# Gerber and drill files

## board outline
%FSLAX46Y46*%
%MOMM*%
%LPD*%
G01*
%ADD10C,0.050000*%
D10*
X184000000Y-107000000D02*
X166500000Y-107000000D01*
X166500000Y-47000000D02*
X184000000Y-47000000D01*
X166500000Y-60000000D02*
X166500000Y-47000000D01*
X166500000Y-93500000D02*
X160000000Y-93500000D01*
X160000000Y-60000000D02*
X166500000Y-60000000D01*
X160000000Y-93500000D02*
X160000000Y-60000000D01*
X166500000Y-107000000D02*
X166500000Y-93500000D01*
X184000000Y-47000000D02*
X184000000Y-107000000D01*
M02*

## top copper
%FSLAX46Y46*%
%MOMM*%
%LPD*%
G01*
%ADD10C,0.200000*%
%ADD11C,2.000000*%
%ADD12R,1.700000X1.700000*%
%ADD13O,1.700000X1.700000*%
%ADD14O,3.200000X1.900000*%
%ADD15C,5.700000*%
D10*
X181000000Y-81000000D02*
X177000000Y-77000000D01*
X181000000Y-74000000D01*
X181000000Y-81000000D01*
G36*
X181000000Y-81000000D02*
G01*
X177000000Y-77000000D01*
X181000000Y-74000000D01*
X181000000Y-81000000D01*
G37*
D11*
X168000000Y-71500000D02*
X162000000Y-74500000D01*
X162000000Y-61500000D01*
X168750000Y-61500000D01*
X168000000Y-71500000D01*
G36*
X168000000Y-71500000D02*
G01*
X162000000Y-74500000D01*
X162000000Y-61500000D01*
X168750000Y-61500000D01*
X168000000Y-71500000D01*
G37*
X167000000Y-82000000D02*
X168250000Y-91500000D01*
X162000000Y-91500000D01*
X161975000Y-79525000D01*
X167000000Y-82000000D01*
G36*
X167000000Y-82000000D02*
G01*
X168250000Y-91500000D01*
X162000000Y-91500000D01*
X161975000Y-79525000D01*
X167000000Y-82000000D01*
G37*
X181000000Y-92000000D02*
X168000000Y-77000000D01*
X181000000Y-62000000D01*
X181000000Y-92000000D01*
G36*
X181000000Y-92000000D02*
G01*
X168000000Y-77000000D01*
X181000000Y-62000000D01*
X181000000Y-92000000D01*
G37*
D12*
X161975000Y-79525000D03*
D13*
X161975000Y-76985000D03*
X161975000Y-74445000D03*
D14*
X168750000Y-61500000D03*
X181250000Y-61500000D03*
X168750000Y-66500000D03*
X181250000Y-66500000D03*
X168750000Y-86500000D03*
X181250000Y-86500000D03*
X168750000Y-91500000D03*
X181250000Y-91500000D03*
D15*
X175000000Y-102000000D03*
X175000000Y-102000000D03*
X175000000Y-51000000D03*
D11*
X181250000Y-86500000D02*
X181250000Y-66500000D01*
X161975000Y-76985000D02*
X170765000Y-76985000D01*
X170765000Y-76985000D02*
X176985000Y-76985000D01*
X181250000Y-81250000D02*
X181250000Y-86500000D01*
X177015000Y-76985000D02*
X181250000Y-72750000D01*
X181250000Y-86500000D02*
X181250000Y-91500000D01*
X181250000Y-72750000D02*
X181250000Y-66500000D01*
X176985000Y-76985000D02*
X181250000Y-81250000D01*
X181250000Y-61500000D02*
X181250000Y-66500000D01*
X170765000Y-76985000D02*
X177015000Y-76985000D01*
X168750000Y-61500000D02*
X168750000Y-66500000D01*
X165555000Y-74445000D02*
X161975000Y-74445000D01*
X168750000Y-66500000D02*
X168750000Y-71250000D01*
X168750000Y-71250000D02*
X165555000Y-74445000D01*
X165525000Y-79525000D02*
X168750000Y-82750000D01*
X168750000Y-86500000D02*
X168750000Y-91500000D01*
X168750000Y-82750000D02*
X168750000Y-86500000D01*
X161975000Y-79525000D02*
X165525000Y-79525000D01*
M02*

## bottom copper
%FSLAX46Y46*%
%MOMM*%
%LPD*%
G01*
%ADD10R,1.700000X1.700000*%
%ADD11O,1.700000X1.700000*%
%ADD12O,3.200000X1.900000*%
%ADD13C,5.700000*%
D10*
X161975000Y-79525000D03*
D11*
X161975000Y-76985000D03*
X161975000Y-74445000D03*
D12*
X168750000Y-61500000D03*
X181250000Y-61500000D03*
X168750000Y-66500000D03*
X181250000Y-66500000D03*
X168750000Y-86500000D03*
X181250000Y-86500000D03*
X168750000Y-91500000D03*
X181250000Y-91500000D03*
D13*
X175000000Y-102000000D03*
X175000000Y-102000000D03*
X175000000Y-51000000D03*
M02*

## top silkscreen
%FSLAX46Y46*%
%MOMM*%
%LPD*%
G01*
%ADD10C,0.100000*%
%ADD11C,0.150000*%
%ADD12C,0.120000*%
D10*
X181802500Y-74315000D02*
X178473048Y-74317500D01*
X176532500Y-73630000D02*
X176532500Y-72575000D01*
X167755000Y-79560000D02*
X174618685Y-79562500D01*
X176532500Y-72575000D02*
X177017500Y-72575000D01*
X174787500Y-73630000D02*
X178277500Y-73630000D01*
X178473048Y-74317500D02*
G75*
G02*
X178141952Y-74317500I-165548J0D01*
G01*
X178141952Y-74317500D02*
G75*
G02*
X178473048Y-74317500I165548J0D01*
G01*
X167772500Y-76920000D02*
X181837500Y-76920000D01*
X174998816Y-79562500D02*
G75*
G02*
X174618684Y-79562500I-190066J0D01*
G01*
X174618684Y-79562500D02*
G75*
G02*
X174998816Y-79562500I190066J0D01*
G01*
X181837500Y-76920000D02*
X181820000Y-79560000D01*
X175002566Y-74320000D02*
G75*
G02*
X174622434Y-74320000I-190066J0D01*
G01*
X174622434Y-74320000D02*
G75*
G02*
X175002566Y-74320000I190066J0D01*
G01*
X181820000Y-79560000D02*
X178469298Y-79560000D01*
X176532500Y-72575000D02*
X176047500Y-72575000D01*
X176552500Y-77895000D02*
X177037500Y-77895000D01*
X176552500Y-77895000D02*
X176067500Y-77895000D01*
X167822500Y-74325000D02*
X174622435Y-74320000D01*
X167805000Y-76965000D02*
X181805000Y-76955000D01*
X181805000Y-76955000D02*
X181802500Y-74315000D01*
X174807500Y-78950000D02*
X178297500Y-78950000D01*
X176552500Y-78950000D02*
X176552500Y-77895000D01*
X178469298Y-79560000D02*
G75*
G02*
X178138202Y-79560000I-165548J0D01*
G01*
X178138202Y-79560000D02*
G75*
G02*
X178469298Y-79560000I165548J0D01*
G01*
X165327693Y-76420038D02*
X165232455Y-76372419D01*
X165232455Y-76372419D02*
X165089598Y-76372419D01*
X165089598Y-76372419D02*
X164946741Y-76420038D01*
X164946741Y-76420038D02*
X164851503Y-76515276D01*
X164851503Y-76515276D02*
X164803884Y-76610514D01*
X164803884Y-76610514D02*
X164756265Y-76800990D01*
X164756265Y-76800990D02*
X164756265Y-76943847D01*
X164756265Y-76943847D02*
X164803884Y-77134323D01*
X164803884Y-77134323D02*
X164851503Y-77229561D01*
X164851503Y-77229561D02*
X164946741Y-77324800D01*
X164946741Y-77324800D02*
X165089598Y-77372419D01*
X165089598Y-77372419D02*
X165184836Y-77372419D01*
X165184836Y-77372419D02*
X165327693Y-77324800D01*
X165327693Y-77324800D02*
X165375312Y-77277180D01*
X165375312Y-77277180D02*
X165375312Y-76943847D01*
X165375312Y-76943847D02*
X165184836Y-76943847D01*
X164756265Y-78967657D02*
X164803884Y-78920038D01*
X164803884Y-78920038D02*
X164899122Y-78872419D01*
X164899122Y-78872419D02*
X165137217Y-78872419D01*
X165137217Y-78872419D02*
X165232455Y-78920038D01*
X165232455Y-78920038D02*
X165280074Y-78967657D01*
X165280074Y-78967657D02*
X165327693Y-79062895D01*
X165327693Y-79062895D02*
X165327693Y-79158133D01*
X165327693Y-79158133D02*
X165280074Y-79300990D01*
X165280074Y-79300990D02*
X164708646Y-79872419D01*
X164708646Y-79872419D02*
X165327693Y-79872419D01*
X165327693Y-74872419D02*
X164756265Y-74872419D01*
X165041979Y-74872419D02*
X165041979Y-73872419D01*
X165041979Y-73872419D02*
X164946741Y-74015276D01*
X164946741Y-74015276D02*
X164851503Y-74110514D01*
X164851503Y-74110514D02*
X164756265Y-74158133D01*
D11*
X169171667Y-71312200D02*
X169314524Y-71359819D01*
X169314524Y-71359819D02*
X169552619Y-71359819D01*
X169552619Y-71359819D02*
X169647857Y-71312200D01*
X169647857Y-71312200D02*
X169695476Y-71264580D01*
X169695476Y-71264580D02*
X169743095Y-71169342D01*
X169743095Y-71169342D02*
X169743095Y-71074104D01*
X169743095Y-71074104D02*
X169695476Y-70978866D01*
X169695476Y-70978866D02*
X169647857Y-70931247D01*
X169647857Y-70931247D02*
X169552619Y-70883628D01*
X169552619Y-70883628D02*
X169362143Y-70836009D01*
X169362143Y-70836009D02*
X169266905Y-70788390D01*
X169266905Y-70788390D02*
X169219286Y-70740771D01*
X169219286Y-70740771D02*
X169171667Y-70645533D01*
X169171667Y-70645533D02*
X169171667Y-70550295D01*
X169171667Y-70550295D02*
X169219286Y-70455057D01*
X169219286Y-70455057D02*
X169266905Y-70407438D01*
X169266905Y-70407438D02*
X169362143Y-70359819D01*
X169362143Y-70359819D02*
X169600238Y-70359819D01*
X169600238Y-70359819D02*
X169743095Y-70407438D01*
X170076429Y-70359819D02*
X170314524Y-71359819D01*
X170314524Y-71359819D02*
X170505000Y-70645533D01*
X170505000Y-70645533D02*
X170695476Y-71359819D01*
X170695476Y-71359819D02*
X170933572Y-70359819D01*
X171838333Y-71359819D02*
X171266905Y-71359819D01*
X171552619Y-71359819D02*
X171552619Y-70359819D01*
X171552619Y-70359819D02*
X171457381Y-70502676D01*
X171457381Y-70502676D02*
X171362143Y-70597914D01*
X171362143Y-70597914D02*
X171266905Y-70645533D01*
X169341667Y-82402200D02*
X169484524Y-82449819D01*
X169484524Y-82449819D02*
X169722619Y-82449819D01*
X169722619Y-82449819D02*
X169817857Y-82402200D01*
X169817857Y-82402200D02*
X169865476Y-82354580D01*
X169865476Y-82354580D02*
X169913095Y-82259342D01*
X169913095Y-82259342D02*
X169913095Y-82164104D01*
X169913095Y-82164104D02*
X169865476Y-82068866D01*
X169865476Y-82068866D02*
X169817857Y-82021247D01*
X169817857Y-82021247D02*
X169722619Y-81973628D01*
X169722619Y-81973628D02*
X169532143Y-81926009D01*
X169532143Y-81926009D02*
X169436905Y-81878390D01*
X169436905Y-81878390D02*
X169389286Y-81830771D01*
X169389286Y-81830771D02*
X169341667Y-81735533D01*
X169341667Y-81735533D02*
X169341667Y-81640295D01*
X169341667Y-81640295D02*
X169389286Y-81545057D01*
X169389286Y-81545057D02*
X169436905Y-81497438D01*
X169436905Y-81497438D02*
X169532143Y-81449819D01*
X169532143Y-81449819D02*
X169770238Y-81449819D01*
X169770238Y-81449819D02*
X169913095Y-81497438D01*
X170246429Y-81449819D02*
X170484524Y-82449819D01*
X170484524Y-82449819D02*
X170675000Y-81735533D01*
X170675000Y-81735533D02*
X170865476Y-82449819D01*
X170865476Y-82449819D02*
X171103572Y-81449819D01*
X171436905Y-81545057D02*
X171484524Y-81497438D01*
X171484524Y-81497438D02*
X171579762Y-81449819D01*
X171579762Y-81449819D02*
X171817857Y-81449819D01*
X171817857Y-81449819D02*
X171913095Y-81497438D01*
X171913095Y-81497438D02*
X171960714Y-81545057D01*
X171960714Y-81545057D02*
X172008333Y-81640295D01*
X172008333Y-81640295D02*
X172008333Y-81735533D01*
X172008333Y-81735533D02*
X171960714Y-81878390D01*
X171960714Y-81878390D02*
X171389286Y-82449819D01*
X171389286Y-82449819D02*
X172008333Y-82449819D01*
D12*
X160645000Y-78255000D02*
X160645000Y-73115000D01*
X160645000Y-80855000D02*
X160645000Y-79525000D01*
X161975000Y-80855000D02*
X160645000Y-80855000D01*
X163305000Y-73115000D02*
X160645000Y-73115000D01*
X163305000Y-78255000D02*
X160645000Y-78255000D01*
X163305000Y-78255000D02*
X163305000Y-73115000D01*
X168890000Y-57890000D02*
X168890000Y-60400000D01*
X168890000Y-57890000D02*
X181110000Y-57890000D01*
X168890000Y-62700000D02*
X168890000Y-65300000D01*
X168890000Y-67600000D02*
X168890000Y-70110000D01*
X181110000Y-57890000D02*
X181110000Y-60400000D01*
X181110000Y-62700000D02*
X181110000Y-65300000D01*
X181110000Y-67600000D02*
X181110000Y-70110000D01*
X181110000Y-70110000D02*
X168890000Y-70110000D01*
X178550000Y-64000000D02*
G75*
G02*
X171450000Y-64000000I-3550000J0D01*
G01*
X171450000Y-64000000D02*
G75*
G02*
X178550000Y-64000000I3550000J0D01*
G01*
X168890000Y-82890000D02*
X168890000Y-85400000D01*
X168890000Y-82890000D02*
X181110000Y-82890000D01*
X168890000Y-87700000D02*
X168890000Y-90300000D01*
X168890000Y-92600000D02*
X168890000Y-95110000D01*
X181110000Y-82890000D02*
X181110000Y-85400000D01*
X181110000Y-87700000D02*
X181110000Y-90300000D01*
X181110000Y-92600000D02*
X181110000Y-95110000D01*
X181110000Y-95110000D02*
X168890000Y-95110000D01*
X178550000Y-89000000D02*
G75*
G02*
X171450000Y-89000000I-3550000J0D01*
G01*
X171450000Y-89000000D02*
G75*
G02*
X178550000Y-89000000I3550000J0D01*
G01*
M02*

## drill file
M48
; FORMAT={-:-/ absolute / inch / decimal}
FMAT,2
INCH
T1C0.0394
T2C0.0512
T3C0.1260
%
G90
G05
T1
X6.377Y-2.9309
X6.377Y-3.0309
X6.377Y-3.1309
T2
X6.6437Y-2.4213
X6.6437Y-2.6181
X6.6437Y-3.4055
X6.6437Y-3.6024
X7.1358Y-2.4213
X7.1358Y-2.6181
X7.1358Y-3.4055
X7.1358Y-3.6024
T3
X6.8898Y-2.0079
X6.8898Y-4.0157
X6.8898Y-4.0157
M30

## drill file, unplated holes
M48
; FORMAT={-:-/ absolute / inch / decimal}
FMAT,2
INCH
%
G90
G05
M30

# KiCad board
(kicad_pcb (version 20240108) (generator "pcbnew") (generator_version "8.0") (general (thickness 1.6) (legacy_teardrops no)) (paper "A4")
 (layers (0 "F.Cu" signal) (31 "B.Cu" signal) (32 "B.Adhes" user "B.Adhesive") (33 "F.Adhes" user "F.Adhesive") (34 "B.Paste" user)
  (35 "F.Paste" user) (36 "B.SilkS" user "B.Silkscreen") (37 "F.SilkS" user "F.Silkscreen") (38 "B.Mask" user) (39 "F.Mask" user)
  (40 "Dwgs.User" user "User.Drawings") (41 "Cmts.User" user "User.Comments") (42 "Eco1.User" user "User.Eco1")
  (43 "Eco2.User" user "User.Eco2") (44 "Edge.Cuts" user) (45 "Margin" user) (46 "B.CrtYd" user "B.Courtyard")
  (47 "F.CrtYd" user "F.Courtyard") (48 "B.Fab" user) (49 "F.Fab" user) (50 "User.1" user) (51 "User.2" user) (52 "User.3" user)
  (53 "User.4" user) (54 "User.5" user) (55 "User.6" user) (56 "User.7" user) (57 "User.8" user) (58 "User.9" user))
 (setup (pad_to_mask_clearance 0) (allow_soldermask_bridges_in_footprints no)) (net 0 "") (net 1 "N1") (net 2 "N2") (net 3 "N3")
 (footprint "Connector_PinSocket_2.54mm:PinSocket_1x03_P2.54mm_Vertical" (layer "F.Cu") (at 161.975 79.525 180)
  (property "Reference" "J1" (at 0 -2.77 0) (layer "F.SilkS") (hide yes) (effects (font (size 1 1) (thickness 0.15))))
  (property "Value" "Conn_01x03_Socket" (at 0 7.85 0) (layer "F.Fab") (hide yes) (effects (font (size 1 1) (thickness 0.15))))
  (fp_line (start 1.33 1.27) (end 1.33 6.41) (stroke (width 0.12) (type solid)) (layer "F.SilkS"))
  (fp_line (start 1.33 -1.33) (end 1.33 0) (stroke (width 0.12) (type solid)) (layer "F.SilkS"))
  (fp_line (start 0 -1.33) (end 1.33 -1.33) (stroke (width 0.12) (type solid)) (layer "F.SilkS"))
  (fp_line (start -1.33 6.41) (end 1.33 6.41) (stroke (width 0.12) (type solid)) (layer "F.SilkS"))
  (fp_line (start -1.33 1.27) (end 1.33 1.27) (stroke (width 0.12) (type solid)) (layer "F.SilkS"))
  (fp_line (start -1.33 1.27) (end -1.33 6.41) (stroke (width 0.12) (type solid)) (layer "F.SilkS"))
  (pad "1" thru_hole rect (at 0 0 180) (size 1.7 1.7) (drill 1) (layers "*.Cu" "*.Mask") (remove_unused_layers no) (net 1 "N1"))
  (pad "2" thru_hole oval (at 0 2.54 180) (size 1.7 1.7) (drill 1) (layers "*.Cu" "*.Mask") (remove_unused_layers no) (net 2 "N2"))
  (pad "3" thru_hole oval (at 0 5.08 180) (size 1.7 1.7) (drill 1) (layers "*.Cu" "*.Mask") (remove_unused_layers no) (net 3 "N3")))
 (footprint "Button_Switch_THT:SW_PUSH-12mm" (layer "F.Cu") (at 168.75 61.5)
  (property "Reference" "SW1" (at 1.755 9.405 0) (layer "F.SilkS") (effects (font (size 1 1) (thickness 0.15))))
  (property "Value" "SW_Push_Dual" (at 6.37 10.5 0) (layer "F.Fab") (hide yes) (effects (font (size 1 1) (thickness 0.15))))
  (fp_line (start 0.14 -3.61) (end 0.14 -1.1) (stroke (width 0.12) (type default)) (layer "F.SilkS"))
  (fp_line (start 0.14 -3.61) (end 12.36 -3.61) (stroke (width 0.12) (type default)) (layer "F.SilkS"))
  (fp_line (start 0.14 1.2) (end 0.14 3.8) (stroke (width 0.12) (type default)) (layer "F.SilkS"))
  (fp_line (start 0.14 6.1) (end 0.14 8.61) (stroke (width 0.12) (type default)) (layer "F.SilkS"))
  (fp_line (start 12.36 -3.61) (end 12.36 -1.1) (stroke (width 0.12) (type default)) (layer "F.SilkS"))
  (fp_line (start 12.36 1.2) (end 12.36 3.8) (stroke (width 0.12) (type default)) (layer "F.SilkS"))
  (fp_line (start 12.36 6.1) (end 12.36 8.61) (stroke (width 0.12) (type default)) (layer "F.SilkS"))
  (fp_line (start 12.36 8.61) (end 0.14 8.61) (stroke (width 0.12) (type default)) (layer "F.SilkS"))
  (fp_circle (center 6.25 2.5) (end 9.8 2.5) (stroke (width 0.12) (type default)) (fill none) (layer "F.SilkS"))
  (pad "1" thru_hole oval (at 0 0) (size 3.2 1.9) (drill 1.3) (layers "*.Cu" "*.Mask") (remove_unused_layers no) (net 3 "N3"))
  (pad "2" thru_hole oval (at 12.5 0) (size 3.2 1.9) (drill 1.3) (layers "*.Cu" "*.Mask") (remove_unused_layers no) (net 2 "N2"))
  (pad "3" thru_hole oval (at 0 5) (size 3.2 1.9) (drill 1.3) (layers "*.Cu" "*.Mask") (remove_unused_layers no) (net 3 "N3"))
  (pad "4" thru_hole oval (at 12.5 5) (size 3.2 1.9) (drill 1.3) (layers "*.Cu" "*.Mask") (remove_unused_layers no) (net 2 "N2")))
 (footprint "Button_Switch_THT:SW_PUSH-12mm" (layer "F.Cu") (at 168.75 86.5)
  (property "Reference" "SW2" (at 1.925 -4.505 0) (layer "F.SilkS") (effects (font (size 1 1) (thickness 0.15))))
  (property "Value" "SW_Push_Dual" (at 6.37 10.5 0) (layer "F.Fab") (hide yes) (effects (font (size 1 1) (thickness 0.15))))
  (fp_line (start 0.14 -3.61) (end 0.14 -1.1) (stroke (width 0.12) (type default)) (layer "F.SilkS"))
  (fp_line (start 0.14 -3.61) (end 12.36 -3.61) (stroke (width 0.12) (type default)) (layer "F.SilkS"))
  (fp_line (start 0.14 1.2) (end 0.14 3.8) (stroke (width 0.12) (type default)) (layer "F.SilkS"))
  (fp_line (start 0.14 6.1) (end 0.14 8.61) (stroke (width 0.12) (type default)) (layer "F.SilkS"))
  (fp_line (start 12.36 -3.61) (end 12.36 -1.1) (stroke (width 0.12) (type default)) (layer "F.SilkS"))
  (fp_line (start 12.36 1.2) (end 12.36 3.8) (stroke (width 0.12) (type default)) (layer "F.SilkS"))
  (fp_line (start 12.36 6.1) (end 12.36 8.61) (stroke (width 0.12) (type default)) (layer "F.SilkS"))
  (fp_line (start 12.36 8.61) (end 0.14 8.61) (stroke (width 0.12) (type default)) (layer "F.SilkS"))
  (fp_circle (center 6.25 2.5) (end 9.8 2.5) (stroke (width 0.12) (type default)) (fill none) (layer "F.SilkS"))
  (pad "1" thru_hole oval (at 0 0) (size 3.2 1.9) (drill 1.3) (layers "*.Cu" "*.Mask") (remove_unused_layers no) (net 1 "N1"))
  (pad "2" thru_hole oval (at 12.5 0) (size 3.2 1.9) (drill 1.3) (layers "*.Cu" "*.Mask") (remove_unused_layers no) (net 2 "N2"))
  (pad "3" thru_hole oval (at 0 5) (size 3.2 1.9) (drill 1.3) (layers "*.Cu" "*.Mask") (remove_unused_layers no) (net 1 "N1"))
  (pad "4" thru_hole oval (at 12.5 5) (size 3.2 1.9) (drill 1.3) (layers "*.Cu" "*.Mask") (remove_unused_layers no) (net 2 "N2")))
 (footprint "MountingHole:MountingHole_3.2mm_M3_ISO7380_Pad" (layer "F.Cu") (at 175 102)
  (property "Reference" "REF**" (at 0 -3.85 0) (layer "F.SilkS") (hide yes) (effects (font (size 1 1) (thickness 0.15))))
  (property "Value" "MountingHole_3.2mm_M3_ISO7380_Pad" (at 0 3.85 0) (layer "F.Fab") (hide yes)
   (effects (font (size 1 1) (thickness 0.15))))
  (pad "1" thru_hole circle (at 0 0) (size 5.7 5.7) (drill 3.2) (layers "*.Cu" "*.Mask") (remove_unused_layers no)))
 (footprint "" (layer "F.Cu") (at 175 102)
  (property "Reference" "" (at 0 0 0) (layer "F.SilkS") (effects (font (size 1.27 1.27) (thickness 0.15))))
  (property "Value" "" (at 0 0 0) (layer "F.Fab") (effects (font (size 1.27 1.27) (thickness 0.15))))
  (pad "1" thru_hole circle (at 0 0) (size 5.7 5.7) (drill 3.2) (layers "*.Cu" "*.Mask") (remove_unused_layers no)))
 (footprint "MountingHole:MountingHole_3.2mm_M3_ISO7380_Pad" (layer "F.Cu") (at 175 51)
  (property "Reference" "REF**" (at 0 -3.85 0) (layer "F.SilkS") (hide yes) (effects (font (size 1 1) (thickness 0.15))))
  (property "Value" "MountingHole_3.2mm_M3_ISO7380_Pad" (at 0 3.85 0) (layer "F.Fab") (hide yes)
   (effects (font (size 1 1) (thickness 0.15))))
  (pad "1" thru_hole circle (at 0 0) (size 5.7 5.7) (drill 3.2) (layers "*.Cu" "*.Mask") (remove_unused_layers no)))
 (gr_poly (pts (xy 181 74) (xy 177 77) (xy 181 81)) (stroke (width 0.2) (type solid)) (fill solid) (layer "F.Cu") (net 2))
 (gr_poly
  (pts (xy 168.75 61.5) (xy 162 61.5) (xy 162 74.5) (xy 168 71.5)) (stroke (width 2) (type solid)) (fill solid) (layer "F.Cu") (net 3))
 (gr_poly
  (pts (xy 168.25 91.5) (xy 162 91.5) (xy 161.975 79.525) (xy 167 82)) (stroke (width 2) (type solid)) (fill solid) (layer "F.Cu") (net 1))
 (gr_poly (pts (xy 181 92) (xy 168 77) (xy 181 62)) (stroke (width 2) (type solid)) (fill solid) (layer "F.Cu") (net 2))
 (gr_line (start 181.8025 74.315) (end 178.473048 74.3175) (stroke (width 0.1) (type default)) (layer "F.SilkS"))
 (gr_line (start 176.5325 73.63) (end 176.5325 72.575) (stroke (width 0.1) (type default)) (layer "F.SilkS"))
 (gr_line (start 167.755 79.56) (end 174.618685 79.5625) (stroke (width 0.1) (type default)) (layer "F.SilkS"))
 (gr_line (start 176.5325 72.575) (end 177.0175 72.575) (stroke (width 0.1) (type default)) (layer "F.SilkS"))
 (gr_line (start 174.7875 73.63) (end 178.2775 73.63) (stroke (width 0.1) (type default)) (layer "F.SilkS"))
 (gr_circle (center 178.3075 74.3175) (end 178.4675 74.275) (stroke (width 0.1) (type default)) (fill none) (layer "F.SilkS"))
 (gr_line (start 167.7725 76.92) (end 181.8375 76.92) (stroke (width 0.1) (type default)) (layer "F.SilkS"))
 (gr_circle (center 174.80875 79.5625) (end 174.99875 79.5675) (stroke (width 0.1) (type default)) (fill none) (layer "F.SilkS"))
 (gr_line (start 181.8375 76.92) (end 181.82 79.56) (stroke (width 0.1) (type default)) (layer "F.SilkS"))
 (gr_circle (center 174.8125 74.32) (end 175.0025 74.325) (stroke (width 0.1) (type default)) (fill none) (layer "F.SilkS"))
 (gr_line (start 181.82 79.56) (end 178.469298 79.56) (stroke (width 0.1) (type default)) (layer "F.SilkS"))
 (gr_line (start 176.5325 72.575) (end 176.0475 72.575) (stroke (width 0.1) (type default)) (layer "F.SilkS"))
 (gr_line (start 176.5525 77.895) (end 177.0375 77.895) (stroke (width 0.1) (type default)) (layer "F.SilkS"))
 (gr_line (start 176.5525 77.895) (end 176.0675 77.895) (stroke (width 0.1) (type default)) (layer "F.SilkS"))
 (gr_line (start 167.8225 74.325) (end 174.622435 74.32) (stroke (width 0.1) (type default)) (layer "F.SilkS"))
 (gr_line (start 167.805 76.965) (end 181.805 76.955) (stroke (width 0.1) (type default)) (layer "F.SilkS"))
 (gr_line (start 181.805 76.955) (end 181.8025 74.315) (stroke (width 0.1) (type default)) (layer "F.SilkS"))
 (gr_line (start 174.8075 78.95) (end 178.2975 78.95) (stroke (width 0.1) (type default)) (layer "F.SilkS"))
 (gr_line (start 176.5525 78.95) (end 176.5525 77.895) (stroke (width 0.1) (type default)) (layer "F.SilkS"))
 (gr_circle (center 178.30375 79.56) (end 178.46375 79.5175) (stroke (width 0.1) (type default)) (fill none) (layer "F.SilkS"))
 (gr_line (start 184 107) (end 166.5 107) (stroke (width 0.05) (type default)) (layer "Edge.Cuts"))
 (gr_line (start 166.5 47) (end 184 47) (stroke (width 0.05) (type default)) (layer "Edge.Cuts"))
 (gr_line (start 166.5 60) (end 166.5 47) (stroke (width 0.05) (type default)) (layer "Edge.Cuts"))
 (gr_line (start 166.5 93.5) (end 160 93.5) (stroke (width 0.05) (type default)) (layer "Edge.Cuts"))
 (gr_line (start 160 60) (end 166.5 60) (stroke (width 0.05) (type default)) (layer "Edge.Cuts"))
 (gr_line (start 160 93.5) (end 160 60) (stroke (width 0.05) (type default)) (layer "Edge.Cuts"))
 (gr_line (start 166.5 107) (end 166.5 93.5) (stroke (width 0.05) (type default)) (layer "Edge.Cuts"))
 (gr_line (start 184 47) (end 184 107) (stroke (width 0.05) (type default)) (layer "Edge.Cuts"))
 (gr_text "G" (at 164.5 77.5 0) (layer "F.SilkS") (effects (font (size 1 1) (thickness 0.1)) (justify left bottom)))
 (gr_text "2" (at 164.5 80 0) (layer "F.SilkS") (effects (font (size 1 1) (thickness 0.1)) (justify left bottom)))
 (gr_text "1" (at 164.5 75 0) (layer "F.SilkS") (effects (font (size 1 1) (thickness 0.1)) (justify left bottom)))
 (segment (start 181.25 86.5) (end 181.25 66.5) (width 2) (layer "F.Cu") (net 2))
 (segment (start 161.975 76.985) (end 170.765 76.985) (width 2) (layer "F.Cu") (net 2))
 (segment (start 170.765 76.985) (end 176.985 76.985) (width 2) (layer "F.Cu") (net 2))
 (segment (start 181.25 81.25) (end 181.25 86.5) (width 2) (layer "F.Cu") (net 2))
 (segment (start 177.015 76.985) (end 181.25 72.75) (width 2) (layer "F.Cu") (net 2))
 (segment (start 181.25 86.5) (end 181.25 91.5) (width 2) (layer "F.Cu") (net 2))
 (segment (start 181.25 72.75) (end 181.25 66.5) (width 2) (layer "F.Cu") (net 2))
 (segment (start 176.985 76.985) (end 181.25 81.25) (width 2) (layer "F.Cu") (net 2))
 (segment (start 181.25 61.5) (end 181.25 66.5) (width 2) (layer "F.Cu") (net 2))
 (segment (start 170.765 76.985) (end 177.015 76.985) (width 2) (layer "F.Cu") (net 2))
 (segment (start 168.75 61.5) (end 168.75 66.5) (width 2) (layer "F.Cu") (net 3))
 (segment (start 165.555 74.445) (end 161.975 74.445) (width 2) (layer "F.Cu") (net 3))
 (segment (start 168.75 66.5) (end 168.75 71.25) (width 2) (layer "F.Cu") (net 3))
 (segment (start 168.75 71.25) (end 165.555 74.445) (width 2) (layer "F.Cu") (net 3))
 (segment (start 165.525 79.525) (end 168.75 82.75) (width 2) (layer "F.Cu") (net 1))
 (segment (start 168.75 86.5) (end 168.75 91.5) (width 2) (layer "F.Cu") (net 1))
 (segment (start 168.75 82.75) (end 168.75 86.5) (width 2) (layer "F.Cu") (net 1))
 (segment (start 161.975 79.525) (end 165.525 79.525) (width 2) (layer "F.Cu") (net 1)))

